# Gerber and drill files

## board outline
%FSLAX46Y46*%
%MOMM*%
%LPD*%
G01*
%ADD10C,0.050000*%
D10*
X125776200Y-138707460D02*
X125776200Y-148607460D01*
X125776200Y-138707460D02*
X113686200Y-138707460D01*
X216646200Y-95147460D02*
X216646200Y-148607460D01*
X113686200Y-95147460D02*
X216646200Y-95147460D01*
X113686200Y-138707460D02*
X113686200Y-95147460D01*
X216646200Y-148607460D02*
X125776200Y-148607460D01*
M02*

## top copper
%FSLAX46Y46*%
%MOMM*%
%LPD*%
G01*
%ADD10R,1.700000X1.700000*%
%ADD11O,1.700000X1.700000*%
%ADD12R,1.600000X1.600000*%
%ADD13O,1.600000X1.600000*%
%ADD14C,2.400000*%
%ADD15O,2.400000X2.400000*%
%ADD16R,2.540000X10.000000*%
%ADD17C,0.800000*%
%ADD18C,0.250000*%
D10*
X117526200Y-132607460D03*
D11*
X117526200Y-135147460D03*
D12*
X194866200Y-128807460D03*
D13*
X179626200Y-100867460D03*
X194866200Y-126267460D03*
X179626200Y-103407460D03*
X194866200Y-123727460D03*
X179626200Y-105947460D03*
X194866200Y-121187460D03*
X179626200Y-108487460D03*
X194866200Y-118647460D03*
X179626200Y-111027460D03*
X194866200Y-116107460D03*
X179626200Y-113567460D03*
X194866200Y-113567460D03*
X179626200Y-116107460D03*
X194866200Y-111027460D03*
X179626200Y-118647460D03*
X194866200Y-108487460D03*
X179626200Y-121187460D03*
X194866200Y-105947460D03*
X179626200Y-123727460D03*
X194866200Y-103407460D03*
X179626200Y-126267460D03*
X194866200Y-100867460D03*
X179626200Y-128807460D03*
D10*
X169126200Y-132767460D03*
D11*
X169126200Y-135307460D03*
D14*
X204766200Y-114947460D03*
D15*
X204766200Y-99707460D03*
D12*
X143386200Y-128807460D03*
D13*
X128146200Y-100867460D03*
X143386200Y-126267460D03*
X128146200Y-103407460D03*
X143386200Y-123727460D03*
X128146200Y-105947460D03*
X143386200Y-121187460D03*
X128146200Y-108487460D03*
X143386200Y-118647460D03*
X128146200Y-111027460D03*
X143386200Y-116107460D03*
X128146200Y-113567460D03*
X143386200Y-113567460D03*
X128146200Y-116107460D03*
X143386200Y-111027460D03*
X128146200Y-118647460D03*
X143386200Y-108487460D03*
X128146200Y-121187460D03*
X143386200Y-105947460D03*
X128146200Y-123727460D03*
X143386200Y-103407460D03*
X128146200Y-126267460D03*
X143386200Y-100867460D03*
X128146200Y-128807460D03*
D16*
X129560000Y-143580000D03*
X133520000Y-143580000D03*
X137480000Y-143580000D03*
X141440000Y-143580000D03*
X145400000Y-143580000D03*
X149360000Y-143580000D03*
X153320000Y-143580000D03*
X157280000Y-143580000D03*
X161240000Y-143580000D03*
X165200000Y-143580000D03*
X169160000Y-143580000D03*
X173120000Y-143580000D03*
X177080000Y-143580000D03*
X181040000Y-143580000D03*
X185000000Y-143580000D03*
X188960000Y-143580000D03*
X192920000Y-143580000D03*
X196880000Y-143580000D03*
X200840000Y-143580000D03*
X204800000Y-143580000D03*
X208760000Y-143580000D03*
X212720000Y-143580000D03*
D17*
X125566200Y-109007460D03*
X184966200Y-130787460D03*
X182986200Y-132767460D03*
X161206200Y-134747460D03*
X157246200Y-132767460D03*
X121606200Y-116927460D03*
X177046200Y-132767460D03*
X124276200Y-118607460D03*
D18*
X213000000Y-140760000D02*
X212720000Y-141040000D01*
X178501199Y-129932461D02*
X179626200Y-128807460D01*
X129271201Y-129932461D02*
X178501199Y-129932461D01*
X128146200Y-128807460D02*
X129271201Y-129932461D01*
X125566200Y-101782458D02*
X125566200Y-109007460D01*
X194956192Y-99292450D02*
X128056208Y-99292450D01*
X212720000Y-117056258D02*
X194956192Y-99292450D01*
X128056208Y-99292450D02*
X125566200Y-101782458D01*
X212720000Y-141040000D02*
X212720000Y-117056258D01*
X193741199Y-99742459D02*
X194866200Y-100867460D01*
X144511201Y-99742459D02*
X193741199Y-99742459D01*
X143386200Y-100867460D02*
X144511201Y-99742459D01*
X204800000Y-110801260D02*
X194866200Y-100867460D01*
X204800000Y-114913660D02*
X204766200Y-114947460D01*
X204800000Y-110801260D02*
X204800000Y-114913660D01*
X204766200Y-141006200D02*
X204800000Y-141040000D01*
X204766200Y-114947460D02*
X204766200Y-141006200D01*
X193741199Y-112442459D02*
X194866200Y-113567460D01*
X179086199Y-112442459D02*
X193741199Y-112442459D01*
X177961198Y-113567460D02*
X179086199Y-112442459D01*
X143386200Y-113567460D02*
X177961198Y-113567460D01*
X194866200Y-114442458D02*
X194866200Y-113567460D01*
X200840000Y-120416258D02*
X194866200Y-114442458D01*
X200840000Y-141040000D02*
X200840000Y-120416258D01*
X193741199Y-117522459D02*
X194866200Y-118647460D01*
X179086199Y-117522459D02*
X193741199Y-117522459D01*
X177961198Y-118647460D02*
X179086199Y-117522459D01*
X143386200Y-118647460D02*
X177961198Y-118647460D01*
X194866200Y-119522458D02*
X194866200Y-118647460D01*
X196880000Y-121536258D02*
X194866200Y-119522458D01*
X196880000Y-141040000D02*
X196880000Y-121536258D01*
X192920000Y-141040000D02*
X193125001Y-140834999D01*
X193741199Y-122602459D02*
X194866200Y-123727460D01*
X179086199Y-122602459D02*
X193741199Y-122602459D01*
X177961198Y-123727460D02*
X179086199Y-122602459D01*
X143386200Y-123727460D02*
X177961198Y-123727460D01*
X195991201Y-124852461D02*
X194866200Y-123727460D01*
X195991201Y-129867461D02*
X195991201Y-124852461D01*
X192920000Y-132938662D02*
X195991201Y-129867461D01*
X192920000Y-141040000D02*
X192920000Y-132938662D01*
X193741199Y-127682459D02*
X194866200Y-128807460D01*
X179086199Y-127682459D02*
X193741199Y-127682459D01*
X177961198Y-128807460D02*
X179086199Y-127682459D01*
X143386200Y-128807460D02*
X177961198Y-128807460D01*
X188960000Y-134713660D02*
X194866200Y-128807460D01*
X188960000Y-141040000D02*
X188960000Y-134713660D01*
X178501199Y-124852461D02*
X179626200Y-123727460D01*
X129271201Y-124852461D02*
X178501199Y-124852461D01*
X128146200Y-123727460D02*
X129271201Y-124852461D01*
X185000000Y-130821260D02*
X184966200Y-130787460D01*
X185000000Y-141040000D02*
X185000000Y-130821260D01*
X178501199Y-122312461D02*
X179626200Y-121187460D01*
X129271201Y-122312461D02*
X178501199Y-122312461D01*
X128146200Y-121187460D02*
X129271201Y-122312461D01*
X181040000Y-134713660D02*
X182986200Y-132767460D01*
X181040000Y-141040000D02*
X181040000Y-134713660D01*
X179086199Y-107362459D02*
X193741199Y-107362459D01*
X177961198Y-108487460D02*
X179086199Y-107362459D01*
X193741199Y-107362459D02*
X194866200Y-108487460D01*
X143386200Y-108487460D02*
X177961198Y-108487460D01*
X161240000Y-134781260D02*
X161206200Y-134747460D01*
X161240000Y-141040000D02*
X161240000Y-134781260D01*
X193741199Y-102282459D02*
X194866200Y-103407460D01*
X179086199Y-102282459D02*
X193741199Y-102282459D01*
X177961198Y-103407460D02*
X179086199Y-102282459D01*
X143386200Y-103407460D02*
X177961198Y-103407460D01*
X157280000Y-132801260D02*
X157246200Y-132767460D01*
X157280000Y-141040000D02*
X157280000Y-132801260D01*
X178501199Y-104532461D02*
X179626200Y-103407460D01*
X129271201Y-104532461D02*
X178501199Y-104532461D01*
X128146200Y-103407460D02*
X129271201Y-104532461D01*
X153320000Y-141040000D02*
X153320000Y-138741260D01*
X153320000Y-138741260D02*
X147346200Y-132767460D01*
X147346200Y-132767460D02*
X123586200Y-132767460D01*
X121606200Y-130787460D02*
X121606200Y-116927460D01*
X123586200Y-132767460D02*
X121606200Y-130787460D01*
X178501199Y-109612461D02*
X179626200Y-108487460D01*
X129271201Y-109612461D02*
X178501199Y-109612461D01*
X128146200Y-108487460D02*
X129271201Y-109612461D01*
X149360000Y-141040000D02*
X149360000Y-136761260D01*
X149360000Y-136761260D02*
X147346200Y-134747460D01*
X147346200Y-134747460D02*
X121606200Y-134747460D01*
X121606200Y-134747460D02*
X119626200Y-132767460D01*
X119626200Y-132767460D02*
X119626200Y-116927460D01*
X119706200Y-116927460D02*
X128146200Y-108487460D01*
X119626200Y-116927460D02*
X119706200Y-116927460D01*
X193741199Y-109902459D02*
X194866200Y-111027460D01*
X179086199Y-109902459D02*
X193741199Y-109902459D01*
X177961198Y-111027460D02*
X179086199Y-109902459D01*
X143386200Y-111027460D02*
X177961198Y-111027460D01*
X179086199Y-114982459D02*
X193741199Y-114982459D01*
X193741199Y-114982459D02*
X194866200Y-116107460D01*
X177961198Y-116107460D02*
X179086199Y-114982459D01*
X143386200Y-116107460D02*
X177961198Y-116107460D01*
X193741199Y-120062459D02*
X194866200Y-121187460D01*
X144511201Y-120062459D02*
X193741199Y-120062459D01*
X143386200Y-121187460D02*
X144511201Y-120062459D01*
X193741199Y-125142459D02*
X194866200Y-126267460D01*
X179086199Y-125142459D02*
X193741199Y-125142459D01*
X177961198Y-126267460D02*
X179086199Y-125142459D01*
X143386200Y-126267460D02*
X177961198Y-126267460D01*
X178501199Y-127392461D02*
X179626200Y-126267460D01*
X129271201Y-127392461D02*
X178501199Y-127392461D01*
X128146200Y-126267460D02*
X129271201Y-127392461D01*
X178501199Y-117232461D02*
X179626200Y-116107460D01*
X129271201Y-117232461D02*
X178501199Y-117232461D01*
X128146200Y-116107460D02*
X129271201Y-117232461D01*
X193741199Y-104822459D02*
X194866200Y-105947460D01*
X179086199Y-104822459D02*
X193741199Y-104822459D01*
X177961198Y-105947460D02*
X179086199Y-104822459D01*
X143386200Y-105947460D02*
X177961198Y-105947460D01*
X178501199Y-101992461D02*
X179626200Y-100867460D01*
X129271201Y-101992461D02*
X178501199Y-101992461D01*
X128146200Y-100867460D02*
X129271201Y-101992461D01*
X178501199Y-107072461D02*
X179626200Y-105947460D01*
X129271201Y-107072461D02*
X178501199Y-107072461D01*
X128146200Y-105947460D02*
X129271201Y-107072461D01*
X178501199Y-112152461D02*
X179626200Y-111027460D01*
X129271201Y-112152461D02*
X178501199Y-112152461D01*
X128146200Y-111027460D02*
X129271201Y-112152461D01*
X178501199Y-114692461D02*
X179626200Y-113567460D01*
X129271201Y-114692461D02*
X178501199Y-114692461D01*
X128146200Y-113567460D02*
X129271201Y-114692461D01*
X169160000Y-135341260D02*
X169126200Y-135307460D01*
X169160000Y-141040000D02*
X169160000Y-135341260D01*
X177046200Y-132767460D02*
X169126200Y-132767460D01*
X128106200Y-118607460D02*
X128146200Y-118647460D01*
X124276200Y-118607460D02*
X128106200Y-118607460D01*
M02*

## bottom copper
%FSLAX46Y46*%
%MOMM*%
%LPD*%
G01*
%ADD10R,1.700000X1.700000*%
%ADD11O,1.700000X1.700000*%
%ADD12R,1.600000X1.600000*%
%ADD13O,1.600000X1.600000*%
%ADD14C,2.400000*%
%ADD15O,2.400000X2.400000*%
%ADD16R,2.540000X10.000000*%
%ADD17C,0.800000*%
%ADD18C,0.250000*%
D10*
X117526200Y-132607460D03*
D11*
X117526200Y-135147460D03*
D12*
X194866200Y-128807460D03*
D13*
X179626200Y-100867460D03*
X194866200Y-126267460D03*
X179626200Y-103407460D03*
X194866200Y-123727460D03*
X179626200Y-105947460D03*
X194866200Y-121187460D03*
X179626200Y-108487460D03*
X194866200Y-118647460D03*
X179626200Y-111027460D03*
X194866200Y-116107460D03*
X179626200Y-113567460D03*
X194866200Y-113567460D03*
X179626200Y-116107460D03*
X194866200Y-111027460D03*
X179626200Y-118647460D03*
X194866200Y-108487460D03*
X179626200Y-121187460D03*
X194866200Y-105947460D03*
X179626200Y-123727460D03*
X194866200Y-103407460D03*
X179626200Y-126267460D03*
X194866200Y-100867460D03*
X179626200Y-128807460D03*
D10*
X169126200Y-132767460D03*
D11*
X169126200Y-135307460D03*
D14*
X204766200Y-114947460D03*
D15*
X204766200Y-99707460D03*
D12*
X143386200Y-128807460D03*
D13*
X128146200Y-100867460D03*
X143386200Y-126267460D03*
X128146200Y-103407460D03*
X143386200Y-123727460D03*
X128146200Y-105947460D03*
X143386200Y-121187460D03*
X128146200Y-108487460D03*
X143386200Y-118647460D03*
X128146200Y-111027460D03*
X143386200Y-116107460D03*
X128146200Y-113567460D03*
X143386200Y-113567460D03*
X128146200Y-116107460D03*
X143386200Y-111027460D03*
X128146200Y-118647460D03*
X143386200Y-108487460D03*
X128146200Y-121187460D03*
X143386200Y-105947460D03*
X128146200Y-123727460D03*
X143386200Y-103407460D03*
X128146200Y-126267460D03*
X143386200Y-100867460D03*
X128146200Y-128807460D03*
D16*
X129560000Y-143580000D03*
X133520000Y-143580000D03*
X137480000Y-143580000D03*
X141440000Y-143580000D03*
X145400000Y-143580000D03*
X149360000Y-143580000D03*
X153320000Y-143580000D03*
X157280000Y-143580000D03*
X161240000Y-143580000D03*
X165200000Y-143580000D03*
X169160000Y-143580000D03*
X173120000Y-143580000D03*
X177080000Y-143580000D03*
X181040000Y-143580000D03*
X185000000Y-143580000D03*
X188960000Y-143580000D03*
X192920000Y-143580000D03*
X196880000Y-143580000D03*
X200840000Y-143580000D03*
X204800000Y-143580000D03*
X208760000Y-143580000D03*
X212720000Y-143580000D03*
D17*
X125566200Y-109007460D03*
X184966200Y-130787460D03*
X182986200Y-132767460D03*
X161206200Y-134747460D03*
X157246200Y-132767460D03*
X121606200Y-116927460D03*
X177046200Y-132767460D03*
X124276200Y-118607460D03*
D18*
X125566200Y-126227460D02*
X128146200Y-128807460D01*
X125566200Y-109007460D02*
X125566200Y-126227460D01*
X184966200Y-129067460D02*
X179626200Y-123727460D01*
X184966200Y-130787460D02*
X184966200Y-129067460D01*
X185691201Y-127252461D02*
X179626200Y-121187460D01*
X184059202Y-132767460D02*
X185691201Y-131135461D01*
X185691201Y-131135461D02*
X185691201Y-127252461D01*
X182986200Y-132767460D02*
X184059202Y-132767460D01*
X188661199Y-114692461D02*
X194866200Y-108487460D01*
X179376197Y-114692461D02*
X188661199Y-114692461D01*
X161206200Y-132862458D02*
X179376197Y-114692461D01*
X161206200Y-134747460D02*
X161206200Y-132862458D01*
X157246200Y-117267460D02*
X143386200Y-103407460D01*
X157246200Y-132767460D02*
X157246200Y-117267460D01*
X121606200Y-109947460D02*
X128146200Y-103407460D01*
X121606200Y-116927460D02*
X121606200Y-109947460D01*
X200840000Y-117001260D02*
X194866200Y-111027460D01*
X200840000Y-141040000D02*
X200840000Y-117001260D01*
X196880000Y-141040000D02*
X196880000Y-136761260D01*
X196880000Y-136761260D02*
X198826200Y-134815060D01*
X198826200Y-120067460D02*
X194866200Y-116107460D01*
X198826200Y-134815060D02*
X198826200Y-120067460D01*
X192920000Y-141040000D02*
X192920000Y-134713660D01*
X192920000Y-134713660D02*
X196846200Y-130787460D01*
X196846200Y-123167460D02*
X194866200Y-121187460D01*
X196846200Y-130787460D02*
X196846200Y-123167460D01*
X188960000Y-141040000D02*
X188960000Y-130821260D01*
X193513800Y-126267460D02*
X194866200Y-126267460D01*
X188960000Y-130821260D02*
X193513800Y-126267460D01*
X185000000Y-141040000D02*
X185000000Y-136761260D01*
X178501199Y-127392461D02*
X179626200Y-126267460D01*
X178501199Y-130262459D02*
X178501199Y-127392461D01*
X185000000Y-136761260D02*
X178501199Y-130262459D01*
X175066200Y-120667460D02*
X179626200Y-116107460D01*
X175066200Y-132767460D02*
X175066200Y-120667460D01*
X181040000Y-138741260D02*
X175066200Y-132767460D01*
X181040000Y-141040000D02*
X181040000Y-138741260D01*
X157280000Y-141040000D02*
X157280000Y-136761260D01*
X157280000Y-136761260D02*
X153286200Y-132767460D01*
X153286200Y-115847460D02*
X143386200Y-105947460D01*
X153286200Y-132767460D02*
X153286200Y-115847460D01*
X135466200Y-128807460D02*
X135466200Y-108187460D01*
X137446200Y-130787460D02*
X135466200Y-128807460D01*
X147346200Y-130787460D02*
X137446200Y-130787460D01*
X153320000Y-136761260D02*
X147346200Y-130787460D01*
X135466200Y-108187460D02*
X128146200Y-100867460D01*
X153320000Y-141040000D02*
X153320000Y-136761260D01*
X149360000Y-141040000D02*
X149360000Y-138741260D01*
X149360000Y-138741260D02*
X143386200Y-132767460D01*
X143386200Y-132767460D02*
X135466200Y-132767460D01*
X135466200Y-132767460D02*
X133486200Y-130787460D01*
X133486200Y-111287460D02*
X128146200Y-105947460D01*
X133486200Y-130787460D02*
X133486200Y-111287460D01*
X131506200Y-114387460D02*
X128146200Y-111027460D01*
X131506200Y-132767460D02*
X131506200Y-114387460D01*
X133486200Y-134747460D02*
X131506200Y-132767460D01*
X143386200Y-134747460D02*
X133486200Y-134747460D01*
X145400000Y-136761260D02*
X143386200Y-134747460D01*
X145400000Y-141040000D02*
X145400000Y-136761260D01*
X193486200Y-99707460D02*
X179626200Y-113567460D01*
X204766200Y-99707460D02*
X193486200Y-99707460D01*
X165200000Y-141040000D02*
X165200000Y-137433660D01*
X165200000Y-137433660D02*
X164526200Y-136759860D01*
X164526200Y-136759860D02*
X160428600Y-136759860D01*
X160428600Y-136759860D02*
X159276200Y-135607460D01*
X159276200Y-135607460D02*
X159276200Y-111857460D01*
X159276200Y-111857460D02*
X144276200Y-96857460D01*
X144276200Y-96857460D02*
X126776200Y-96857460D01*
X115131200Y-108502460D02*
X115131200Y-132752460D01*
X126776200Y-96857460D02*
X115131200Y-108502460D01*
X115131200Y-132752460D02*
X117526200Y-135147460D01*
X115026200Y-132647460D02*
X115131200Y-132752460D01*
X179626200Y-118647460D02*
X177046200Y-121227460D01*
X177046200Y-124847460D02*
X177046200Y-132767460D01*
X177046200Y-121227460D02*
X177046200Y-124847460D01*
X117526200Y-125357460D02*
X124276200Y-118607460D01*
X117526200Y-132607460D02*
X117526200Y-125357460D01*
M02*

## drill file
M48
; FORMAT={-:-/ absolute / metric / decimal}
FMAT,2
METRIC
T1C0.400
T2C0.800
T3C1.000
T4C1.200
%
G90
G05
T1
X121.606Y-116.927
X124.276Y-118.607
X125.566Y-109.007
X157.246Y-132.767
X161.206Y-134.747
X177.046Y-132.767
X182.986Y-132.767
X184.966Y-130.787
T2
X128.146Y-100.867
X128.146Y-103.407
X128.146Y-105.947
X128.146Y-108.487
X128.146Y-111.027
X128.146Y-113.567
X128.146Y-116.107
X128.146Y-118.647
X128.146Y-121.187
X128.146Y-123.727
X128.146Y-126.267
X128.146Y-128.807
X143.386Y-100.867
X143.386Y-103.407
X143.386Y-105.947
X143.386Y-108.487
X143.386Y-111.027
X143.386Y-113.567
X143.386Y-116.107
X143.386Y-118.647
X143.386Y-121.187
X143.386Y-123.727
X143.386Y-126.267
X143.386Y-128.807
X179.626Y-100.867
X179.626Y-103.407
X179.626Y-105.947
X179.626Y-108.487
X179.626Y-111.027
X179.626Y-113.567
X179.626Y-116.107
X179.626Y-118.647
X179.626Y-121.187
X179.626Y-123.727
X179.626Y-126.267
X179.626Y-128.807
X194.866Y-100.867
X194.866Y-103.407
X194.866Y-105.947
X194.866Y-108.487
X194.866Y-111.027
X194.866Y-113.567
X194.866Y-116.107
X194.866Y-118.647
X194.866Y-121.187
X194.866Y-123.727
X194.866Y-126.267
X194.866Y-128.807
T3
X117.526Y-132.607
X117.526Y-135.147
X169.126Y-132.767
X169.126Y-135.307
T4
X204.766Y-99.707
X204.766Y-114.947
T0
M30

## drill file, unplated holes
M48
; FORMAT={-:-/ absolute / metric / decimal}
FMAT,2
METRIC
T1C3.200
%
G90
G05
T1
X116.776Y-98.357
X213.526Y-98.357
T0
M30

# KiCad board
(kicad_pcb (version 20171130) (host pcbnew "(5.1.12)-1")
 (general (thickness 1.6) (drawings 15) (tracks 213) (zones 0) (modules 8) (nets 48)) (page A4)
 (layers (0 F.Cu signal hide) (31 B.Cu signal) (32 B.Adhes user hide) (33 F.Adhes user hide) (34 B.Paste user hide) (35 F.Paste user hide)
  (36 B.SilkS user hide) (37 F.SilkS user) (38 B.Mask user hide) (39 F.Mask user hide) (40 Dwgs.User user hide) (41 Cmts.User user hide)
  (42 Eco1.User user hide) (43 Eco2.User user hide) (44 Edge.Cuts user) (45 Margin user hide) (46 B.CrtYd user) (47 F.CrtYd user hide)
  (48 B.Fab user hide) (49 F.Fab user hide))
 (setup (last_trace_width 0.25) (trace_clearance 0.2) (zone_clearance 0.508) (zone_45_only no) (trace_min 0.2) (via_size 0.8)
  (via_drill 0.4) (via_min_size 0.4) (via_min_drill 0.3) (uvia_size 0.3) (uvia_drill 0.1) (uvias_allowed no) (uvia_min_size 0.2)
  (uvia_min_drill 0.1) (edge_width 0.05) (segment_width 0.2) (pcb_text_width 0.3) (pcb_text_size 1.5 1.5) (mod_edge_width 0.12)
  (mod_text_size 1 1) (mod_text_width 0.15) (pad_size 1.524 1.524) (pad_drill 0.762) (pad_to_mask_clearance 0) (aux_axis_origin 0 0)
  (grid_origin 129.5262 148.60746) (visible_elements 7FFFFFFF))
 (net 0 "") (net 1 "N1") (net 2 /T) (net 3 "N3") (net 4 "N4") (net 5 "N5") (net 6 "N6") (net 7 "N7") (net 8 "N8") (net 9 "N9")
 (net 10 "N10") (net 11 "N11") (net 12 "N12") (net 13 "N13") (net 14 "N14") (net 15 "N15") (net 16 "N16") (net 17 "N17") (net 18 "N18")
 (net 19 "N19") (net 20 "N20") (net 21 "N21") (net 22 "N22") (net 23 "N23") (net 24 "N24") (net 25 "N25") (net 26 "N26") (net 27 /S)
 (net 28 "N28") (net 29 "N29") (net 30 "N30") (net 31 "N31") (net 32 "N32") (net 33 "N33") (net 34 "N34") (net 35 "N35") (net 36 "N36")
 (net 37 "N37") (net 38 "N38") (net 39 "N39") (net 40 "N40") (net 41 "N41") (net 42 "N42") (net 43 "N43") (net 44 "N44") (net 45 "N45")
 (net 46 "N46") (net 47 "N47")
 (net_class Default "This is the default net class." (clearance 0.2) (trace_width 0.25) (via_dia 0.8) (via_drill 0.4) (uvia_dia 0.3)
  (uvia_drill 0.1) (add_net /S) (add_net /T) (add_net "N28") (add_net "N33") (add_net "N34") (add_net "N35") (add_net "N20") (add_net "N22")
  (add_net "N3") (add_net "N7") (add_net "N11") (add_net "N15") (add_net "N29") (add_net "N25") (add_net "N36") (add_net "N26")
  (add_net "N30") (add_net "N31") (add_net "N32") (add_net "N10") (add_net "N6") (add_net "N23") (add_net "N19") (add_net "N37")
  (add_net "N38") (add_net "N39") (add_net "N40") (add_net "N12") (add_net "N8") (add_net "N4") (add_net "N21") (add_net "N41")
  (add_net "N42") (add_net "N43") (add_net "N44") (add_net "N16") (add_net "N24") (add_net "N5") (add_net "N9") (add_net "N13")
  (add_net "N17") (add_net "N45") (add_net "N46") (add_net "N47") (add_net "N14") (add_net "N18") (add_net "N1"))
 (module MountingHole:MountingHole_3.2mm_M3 (layer F.Cu) (at 213.5262 98.35746)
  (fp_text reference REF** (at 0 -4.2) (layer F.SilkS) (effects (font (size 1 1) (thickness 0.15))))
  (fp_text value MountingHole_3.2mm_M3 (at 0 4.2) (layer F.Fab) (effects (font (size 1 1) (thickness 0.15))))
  (pad 1 np_thru_hole circle (at 0 0) (size 3.2 3.2) (drill 3.2) (layers *.Cu *.Mask)))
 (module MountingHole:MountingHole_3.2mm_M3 (layer F.Cu) (at 116.7762 98.35746)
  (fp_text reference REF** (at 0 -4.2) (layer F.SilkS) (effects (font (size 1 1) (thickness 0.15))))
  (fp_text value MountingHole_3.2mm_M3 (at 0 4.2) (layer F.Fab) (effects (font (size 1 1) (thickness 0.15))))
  (pad 1 np_thru_hole circle (at 0 0) (size 3.2 3.2) (drill 3.2) (layers *.Cu *.Mask)))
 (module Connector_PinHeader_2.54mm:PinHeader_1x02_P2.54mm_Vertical (layer F.Cu) (at 117.5262 132.60746)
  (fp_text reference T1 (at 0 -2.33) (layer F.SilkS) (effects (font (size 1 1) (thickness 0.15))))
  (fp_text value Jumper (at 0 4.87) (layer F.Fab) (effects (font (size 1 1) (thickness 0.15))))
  (pad 1 thru_hole rect (at 0 0) (size 1.7 1.7) (drill 1) (layers *.Cu *.Mask) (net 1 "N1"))
  (pad 2 thru_hole oval (at 0 2.54) (size 1.7 1.7) (drill 1) (layers *.Cu *.Mask) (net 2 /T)))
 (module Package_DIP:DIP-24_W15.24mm (layer F.Cu) (at 194.8662 128.80746 180)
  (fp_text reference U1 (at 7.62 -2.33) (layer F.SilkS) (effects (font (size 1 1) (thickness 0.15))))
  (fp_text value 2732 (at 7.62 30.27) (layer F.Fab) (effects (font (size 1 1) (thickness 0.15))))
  (pad 1 thru_hole rect (at 0 0 180) (size 1.6 1.6) (drill 0.8) (layers *.Cu *.Mask) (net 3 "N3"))
  (pad 13 thru_hole oval (at 15.24 27.94 180) (size 1.6 1.6) (drill 0.8) (layers *.Cu *.Mask) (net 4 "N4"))
  (pad 2 thru_hole oval (at 0 2.54 180) (size 1.6 1.6) (drill 0.8) (layers *.Cu *.Mask) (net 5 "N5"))
  (pad 14 thru_hole oval (at 15.24 25.4 180) (size 1.6 1.6) (drill 0.8) (layers *.Cu *.Mask) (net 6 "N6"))
  (pad 3 thru_hole oval (at 0 5.08 180) (size 1.6 1.6) (drill 0.8) (layers *.Cu *.Mask) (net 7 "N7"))
  (pad 15 thru_hole oval (at 15.24 22.86 180) (size 1.6 1.6) (drill 0.8) (layers *.Cu *.Mask) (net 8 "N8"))
  (pad 4 thru_hole oval (at 0 7.62 180) (size 1.6 1.6) (drill 0.8) (layers *.Cu *.Mask) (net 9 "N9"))
  (pad 16 thru_hole oval (at 15.24 20.32 180) (size 1.6 1.6) (drill 0.8) (layers *.Cu *.Mask) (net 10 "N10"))
  (pad 5 thru_hole oval (at 0 10.16 180) (size 1.6 1.6) (drill 0.8) (layers *.Cu *.Mask) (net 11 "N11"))
  (pad 17 thru_hole oval (at 15.24 17.78 180) (size 1.6 1.6) (drill 0.8) (layers *.Cu *.Mask) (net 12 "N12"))
  (pad 6 thru_hole oval (at 0 12.7 180) (size 1.6 1.6) (drill 0.8) (layers *.Cu *.Mask) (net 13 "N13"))
  (pad 18 thru_hole oval (at 15.24 15.24 180) (size 1.6 1.6) (drill 0.8) (layers *.Cu *.Mask) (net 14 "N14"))
  (pad 7 thru_hole oval (at 0 15.24 180) (size 1.6 1.6) (drill 0.8) (layers *.Cu *.Mask) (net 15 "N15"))
  (pad 19 thru_hole oval (at 15.24 12.7 180) (size 1.6 1.6) (drill 0.8) (layers *.Cu *.Mask) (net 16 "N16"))
  (pad 8 thru_hole oval (at 0 17.78 180) (size 1.6 1.6) (drill 0.8) (layers *.Cu *.Mask) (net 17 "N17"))
  (pad 20 thru_hole oval (at 15.24 10.16 180) (size 1.6 1.6) (drill 0.8) (layers *.Cu *.Mask) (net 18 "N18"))
  (pad 9 thru_hole oval (at 0 20.32 180) (size 1.6 1.6) (drill 0.8) (layers *.Cu *.Mask) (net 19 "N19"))
  (pad 21 thru_hole oval (at 15.24 7.62 180) (size 1.6 1.6) (drill 0.8) (layers *.Cu *.Mask) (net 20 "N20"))
  (pad 10 thru_hole oval (at 0 22.86 180) (size 1.6 1.6) (drill 0.8) (layers *.Cu *.Mask) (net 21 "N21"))
  (pad 22 thru_hole oval (at 15.24 5.08 180) (size 1.6 1.6) (drill 0.8) (layers *.Cu *.Mask) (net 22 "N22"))
  (pad 11 thru_hole oval (at 0 25.4 180) (size 1.6 1.6) (drill 0.8) (layers *.Cu *.Mask) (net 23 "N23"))
  (pad 23 thru_hole oval (at 15.24 2.54 180) (size 1.6 1.6) (drill 0.8) (layers *.Cu *.Mask) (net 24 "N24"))
  (pad 12 thru_hole oval (at 0 27.94 180) (size 1.6 1.6) (drill 0.8) (layers *.Cu *.Mask) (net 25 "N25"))
  (pad 24 thru_hole oval (at 15.24 0 180) (size 1.6 1.6) (drill 0.8) (layers *.Cu *.Mask) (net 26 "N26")))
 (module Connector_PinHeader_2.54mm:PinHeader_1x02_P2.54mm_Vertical (layer F.Cu) (at 169.1262 132.76746)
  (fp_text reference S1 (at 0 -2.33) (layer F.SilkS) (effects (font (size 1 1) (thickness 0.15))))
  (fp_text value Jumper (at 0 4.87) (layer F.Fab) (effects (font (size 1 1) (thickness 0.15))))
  (pad 1 thru_hole rect (at 0 0) (size 1.7 1.7) (drill 1) (layers *.Cu *.Mask) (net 18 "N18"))
  (pad 2 thru_hole oval (at 0 2.54) (size 1.7 1.7) (drill 1) (layers *.Cu *.Mask) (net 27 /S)))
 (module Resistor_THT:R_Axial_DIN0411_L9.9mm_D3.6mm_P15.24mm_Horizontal (layer F.Cu) (at 204.7662 114.94746 90)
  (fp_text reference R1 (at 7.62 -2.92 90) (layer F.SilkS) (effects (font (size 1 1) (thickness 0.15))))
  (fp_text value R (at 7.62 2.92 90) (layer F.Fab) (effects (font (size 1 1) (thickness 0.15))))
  (pad 1 thru_hole circle (at 0 0 90) (size 2.4 2.4) (drill 1.2) (layers *.Cu *.Mask) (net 25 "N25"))
  (pad 2 thru_hole oval (at 15.24 0 90) (size 2.4 2.4) (drill 1.2) (layers *.Cu *.Mask) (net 14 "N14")))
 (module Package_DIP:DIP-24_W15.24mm (layer F.Cu) (at 143.3862 128.80746 180)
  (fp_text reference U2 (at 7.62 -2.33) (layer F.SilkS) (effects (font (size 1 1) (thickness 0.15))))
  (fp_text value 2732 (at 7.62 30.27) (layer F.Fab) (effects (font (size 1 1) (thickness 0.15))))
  (pad 1 thru_hole rect (at 0 0 180) (size 1.6 1.6) (drill 0.8) (layers *.Cu *.Mask) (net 3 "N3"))
  (pad 13 thru_hole oval (at 15.24 27.94 180) (size 1.6 1.6) (drill 0.8) (layers *.Cu *.Mask) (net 4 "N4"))
  (pad 2 thru_hole oval (at 0 2.54 180) (size 1.6 1.6) (drill 0.8) (layers *.Cu *.Mask) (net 5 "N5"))
  (pad 14 thru_hole oval (at 15.24 25.4 180) (size 1.6 1.6) (drill 0.8) (layers *.Cu *.Mask) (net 6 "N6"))
  (pad 3 thru_hole oval (at 0 5.08 180) (size 1.6 1.6) (drill 0.8) (layers *.Cu *.Mask) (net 7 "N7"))
  (pad 15 thru_hole oval (at 15.24 22.86 180) (size 1.6 1.6) (drill 0.8) (layers *.Cu *.Mask) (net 8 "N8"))
  (pad 4 thru_hole oval (at 0 7.62 180) (size 1.6 1.6) (drill 0.8) (layers *.Cu *.Mask) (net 9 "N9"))
  (pad 16 thru_hole oval (at 15.24 20.32 180) (size 1.6 1.6) (drill 0.8) (layers *.Cu *.Mask) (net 10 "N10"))
  (pad 5 thru_hole oval (at 0 10.16 180) (size 1.6 1.6) (drill 0.8) (layers *.Cu *.Mask) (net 11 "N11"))
  (pad 17 thru_hole oval (at 15.24 17.78 180) (size 1.6 1.6) (drill 0.8) (layers *.Cu *.Mask) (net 12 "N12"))
  (pad 6 thru_hole oval (at 0 12.7 180) (size 1.6 1.6) (drill 0.8) (layers *.Cu *.Mask) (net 13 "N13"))
  (pad 18 thru_hole oval (at 15.24 15.24 180) (size 1.6 1.6) (drill 0.8) (layers *.Cu *.Mask) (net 14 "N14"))
  (pad 7 thru_hole oval (at 0 15.24 180) (size 1.6 1.6) (drill 0.8) (layers *.Cu *.Mask) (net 15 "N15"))
  (pad 19 thru_hole oval (at 15.24 12.7 180) (size 1.6 1.6) (drill 0.8) (layers *.Cu *.Mask) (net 16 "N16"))
  (pad 8 thru_hole oval (at 0 17.78 180) (size 1.6 1.6) (drill 0.8) (layers *.Cu *.Mask) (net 17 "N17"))
  (pad 20 thru_hole oval (at 15.24 10.16 180) (size 1.6 1.6) (drill 0.8) (layers *.Cu *.Mask) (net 1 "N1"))
  (pad 9 thru_hole oval (at 0 20.32 180) (size 1.6 1.6) (drill 0.8) (layers *.Cu *.Mask) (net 19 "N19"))
  (pad 21 thru_hole oval (at 15.24 7.62 180) (size 1.6 1.6) (drill 0.8) (layers *.Cu *.Mask) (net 20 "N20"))
  (pad 10 thru_hole oval (at 0 22.86 180) (size 1.6 1.6) (drill 0.8) (layers *.Cu *.Mask) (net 21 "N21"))
  (pad 22 thru_hole oval (at 15.24 5.08 180) (size 1.6 1.6) (drill 0.8) (layers *.Cu *.Mask) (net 22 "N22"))
  (pad 11 thru_hole oval (at 0 25.4 180) (size 1.6 1.6) (drill 0.8) (layers *.Cu *.Mask) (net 23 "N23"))
  (pad 23 thru_hole oval (at 15.24 2.54 180) (size 1.6 1.6) (drill 0.8) (layers *.Cu *.Mask) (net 24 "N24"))
  (pad 12 thru_hole oval (at 0 27.94 180) (size 1.6 1.6) (drill 0.8) (layers *.Cu *.Mask) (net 25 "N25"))
  (pad 24 thru_hole oval (at 15.24 0 180) (size 1.6 1.6) (drill 0.8) (layers *.Cu *.Mask) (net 26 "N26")))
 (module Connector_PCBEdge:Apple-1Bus (layer F.Cu) (at 185 145)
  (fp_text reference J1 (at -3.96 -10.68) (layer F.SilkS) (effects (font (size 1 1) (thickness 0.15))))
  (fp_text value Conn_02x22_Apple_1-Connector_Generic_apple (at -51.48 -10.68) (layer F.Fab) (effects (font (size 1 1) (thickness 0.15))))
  (pad 1 connect rect (at -55.44 -3.96) (size 2.54 10) (drill (offset 0 2.54)) (layers F.Cu F.Mask) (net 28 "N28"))
  (pad 2 connect rect (at -51.48 -3.96) (size 2.54 10) (drill (offset 0 2.54)) (layers F.Cu F.Mask) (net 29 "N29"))
  (pad 3 connect rect (at -47.52 -3.96) (size 2.54 10) (drill (offset 0 2.54)) (layers F.Cu F.Mask) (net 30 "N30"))
  (pad 4 connect rect (at -43.56 -3.96) (size 2.54 10) (drill (offset 0 2.54)) (layers F.Cu F.Mask) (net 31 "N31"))
  (pad 5 connect rect (at -39.6 -3.96) (size 2.54 10) (drill (offset 0 2.54)) (layers F.Cu F.Mask) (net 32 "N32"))
  (pad 6 connect rect (at -35.64 -3.96) (size 2.54 10) (drill (offset 0 2.54)) (layers F.Cu F.Mask) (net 10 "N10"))
  (pad 7 connect rect (at -31.68 -3.96) (size 2.54 10) (drill (offset 0 2.54)) (layers F.Cu F.Mask) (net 6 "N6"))
  (pad 8 connect rect (at -27.72 -3.96) (size 2.54 10) (drill (offset 0 2.54)) (layers F.Cu F.Mask) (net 23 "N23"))
  (pad 9 connect rect (at -23.76 -3.96) (size 2.54 10) (drill (offset 0 2.54)) (layers F.Cu F.Mask) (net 19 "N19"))
  (pad 10 connect rect (at -19.8 -3.96) (size 2.54 10) (drill (offset 0 2.54)) (layers F.Cu F.Mask) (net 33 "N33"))
  (pad 11 connect rect (at -15.84 -3.96) (size 2.54 10) (drill (offset 0 2.54)) (layers F.Cu F.Mask) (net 27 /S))
  (pad 12 connect rect (at -11.88 -3.96) (size 2.54 10) (drill (offset 0 2.54)) (layers F.Cu F.Mask) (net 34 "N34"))
  (pad 13 connect rect (at -7.92 -3.96) (size 2.54 10) (drill (offset 0 2.54)) (layers F.Cu F.Mask) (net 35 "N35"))
  (pad 14 connect rect (at -3.96 -3.96) (size 2.54 10) (drill (offset 0 2.54)) (layers F.Cu F.Mask) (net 20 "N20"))
  (pad 15 connect rect (at 0 -3.96) (size 2.54 10) (drill (offset 0 2.54)) (layers F.Cu F.Mask) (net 22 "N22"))
  (pad 16 connect rect (at 3.96 -3.96) (size 2.54 10) (drill (offset 0 2.54)) (layers F.Cu F.Mask) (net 3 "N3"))
  (pad 17 connect rect (at 7.92 -3.96) (size 2.54 10) (drill (offset 0 2.54)) (layers F.Cu F.Mask) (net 7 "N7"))
  (pad 18 connect rect (at 11.88 -3.96) (size 2.54 10) (drill (offset 0 2.54)) (layers F.Cu F.Mask) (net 11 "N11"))
  (pad 19 connect rect (at 15.84 -3.96) (size 2.54 10) (drill (offset 0 2.54)) (layers F.Cu F.Mask) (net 15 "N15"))
  (pad 20 connect rect (at 19.8 -3.96) (size 2.54 10) (drill (offset 0 2.54)) (layers F.Cu F.Mask) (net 25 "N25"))
  (pad 21 connect rect (at 23.76 -3.96) (size 2.54 10) (drill (offset 0 2.54)) (layers F.Cu F.Mask) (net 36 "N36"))
  (pad 22 connect rect (at 27.72 -3.96) (size 2.54 10) (drill (offset 0 2.54)) (layers F.Cu F.Mask) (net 26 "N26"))
  (pad A connect rect (at -55.44 -3.96) (size 2.54 10) (drill (offset 0 2.54)) (layers B.Cu B.Mask) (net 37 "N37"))
  (pad B connect rect (at -51.48 -3.96) (size 2.54 10) (drill (offset 0 2.54)) (layers B.Cu B.Mask) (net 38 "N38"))
  (pad C connect rect (at -47.52 -3.96) (size 2.54 10) (drill (offset 0 2.54)) (layers B.Cu B.Mask) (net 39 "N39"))
  (pad D connect rect (at -43.56 -3.96) (size 2.54 10) (drill (offset 0 2.54)) (layers B.Cu B.Mask) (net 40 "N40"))
  (pad E connect rect (at -39.6 -3.96) (size 2.54 10) (drill (offset 0 2.54)) (layers B.Cu B.Mask) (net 12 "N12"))
  (pad F connect rect (at -35.64 -3.96) (size 2.54 10) (drill (offset 0 2.54)) (layers B.Cu B.Mask) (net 8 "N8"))
  (pad H connect rect (at -31.68 -3.96) (size 2.54 10) (drill (offset 0 2.54)) (layers B.Cu B.Mask) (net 4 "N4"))
  (pad J connect rect (at -27.72 -3.96) (size 2.54 10) (drill (offset 0 2.54)) (layers B.Cu B.Mask) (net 21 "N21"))
  (pad K connect rect (at -23.76 -3.96) (size 2.54 10) (drill (offset 0 2.54)) (layers B.Cu B.Mask) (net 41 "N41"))
  (pad L connect rect (at -19.8 -3.96) (size 2.54 10) (drill (offset 0 2.54)) (layers B.Cu B.Mask) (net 2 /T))
  (pad M connect rect (at -15.84 -3.96) (size 2.54 10) (drill (offset 0 2.54)) (layers B.Cu B.Mask) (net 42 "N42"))
  (pad N connect rect (at -11.88 -3.96) (size 2.54 10) (drill (offset 0 2.54)) (layers B.Cu B.Mask) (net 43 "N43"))
  (pad P connect rect (at -7.92 -3.96) (size 2.54 10) (drill (offset 0 2.54)) (layers B.Cu B.Mask) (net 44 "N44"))
  (pad R connect rect (at -3.96 -3.96) (size 2.54 10) (drill (offset 0 2.54)) (layers B.Cu B.Mask) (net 16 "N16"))
  (pad S connect rect (at 0 -3.96) (size 2.54 10) (drill (offset 0 2.54)) (layers B.Cu B.Mask) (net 24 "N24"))
  (pad T connect rect (at 3.96 -3.96) (size 2.54 10) (drill (offset 0 2.54)) (layers B.Cu B.Mask) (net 5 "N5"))
  (pad U connect rect (at 7.92 -3.96) (size 2.54 10) (drill (offset 0 2.54)) (layers B.Cu B.Mask) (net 9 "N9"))
  (pad V connect rect (at 11.88 -3.96) (size 2.54 10) (drill (offset 0 2.54)) (layers B.Cu B.Mask) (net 13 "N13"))
  (pad W connect rect (at 15.84 -3.96) (size 2.54 10) (drill (offset 0 2.54)) (layers B.Cu B.Mask) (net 17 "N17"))
  (pad X connect rect (at 19.8 -3.96) (size 2.54 10) (drill (offset 0 2.54)) (layers B.Cu B.Mask) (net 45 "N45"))
  (pad Y connect rect (at 23.76 -3.96) (size 2.54 10) (drill (offset 0 2.54)) (layers B.Cu B.Mask) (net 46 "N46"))
  (pad Z connect rect (at 27.72 -3.96) (size 2.54 10) (drill (offset 0 2.54)) (layers B.Cu B.Mask) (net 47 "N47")))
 (gr_line (start 125.7762 138.70746) (end 125.7762 148.60746) (layer Edge.Cuts) (width 0.05))
 (gr_line (start 125.7762 138.70746) (end 113.6862 138.70746) (layer Edge.Cuts) (width 0.05))
 (gr_line (start 216.6462 95.14746) (end 216.6462 148.60746) (layer Edge.Cuts) (width 0.05))
 (gr_line (start 113.6862 95.14746) (end 216.6462 95.14746) (layer Edge.Cuts) (width 0.05))
 (gr_line (start 113.6862 138.70746) (end 113.6862 95.14746) (layer Edge.Cuts) (width 0.05))
 (gr_line (start 216.6462 148.60746) (end 125.7762 148.60746) (layer Edge.Cuts) (width 0.05))
 (segment (start 213 140.76) (end 212.72 141.04) (width 0.25) (layer F.Cu) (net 26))
 (segment (start 178.501199 129.932461) (end 179.6262 128.80746) (width 0.25) (layer F.Cu) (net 26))
 (segment (start 129.271201 129.932461) (end 178.501199 129.932461) (width 0.25) (layer F.Cu) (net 26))
 (segment (start 128.1462 128.80746) (end 129.271201 129.932461) (width 0.25) (layer F.Cu) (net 26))
 (via (at 125.5662 109.00746) (size 0.8) (drill 0.4) (layers F.Cu B.Cu) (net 26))
 (segment (start 125.5662 101.782458) (end 125.5662 109.00746) (width 0.25) (layer F.Cu) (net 26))
 (segment (start 194.956192 99.29245) (end 128.056208 99.29245) (width 0.25) (layer F.Cu) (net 26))
 (segment (start 212.72 117.056258) (end 194.956192 99.29245) (width 0.25) (layer F.Cu) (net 26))
 (segment (start 128.056208 99.29245) (end 125.5662 101.782458) (width 0.25) (layer F.Cu) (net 26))
 (segment (start 212.72 141.04) (end 212.72 117.056258) (width 0.25) (layer F.Cu) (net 26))
 (segment (start 125.5662 126.22746) (end 128.1462 128.80746) (width 0.25) (layer B.Cu) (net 26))
 (segment (start 125.5662 109.00746) (end 125.5662 126.22746) (width 0.25) (layer B.Cu) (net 26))
 (segment (start 193.741199 99.742459) (end 194.8662 100.86746) (width 0.25) (layer F.Cu) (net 25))
 (segment (start 144.511201 99.742459) (end 193.741199 99.742459) (width 0.25) (layer F.Cu) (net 25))
 (segment (start 143.3862 100.86746) (end 144.511201 99.742459) (width 0.25) (layer F.Cu) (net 25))
 (segment (start 204.8 110.80126) (end 194.8662 100.86746) (width 0.25) (layer F.Cu) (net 25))
 (segment (start 204.8 114.91366) (end 204.7662 114.94746) (width 0.25) (layer F.Cu) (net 25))
 (segment (start 204.8 110.80126) (end 204.8 114.91366) (width 0.25) (layer F.Cu) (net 25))
 (segment (start 204.7662 141.0062) (end 204.8 141.04) (width 0.25) (layer F.Cu) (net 25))
 (segment (start 204.7662 114.94746) (end 204.7662 141.0062) (width 0.25) (layer F.Cu) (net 25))
 (segment (start 193.741199 112.442459) (end 194.8662 113.56746) (width 0.25) (layer F.Cu) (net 15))
 (segment (start 179.086199 112.442459) (end 193.741199 112.442459) (width 0.25) (layer F.Cu) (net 15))
 (segment (start 177.961198 113.56746) (end 179.086199 112.442459) (width 0.25) (layer F.Cu) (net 15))
 (segment (start 143.3862 113.56746) (end 177.961198 113.56746) (width 0.25) (layer F.Cu) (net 15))
 (segment (start 194.8662 114.442458) (end 194.8662 113.56746) (width 0.25) (layer F.Cu) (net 15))
 (segment (start 200.84 120.416258) (end 194.8662 114.442458) (width 0.25) (layer F.Cu) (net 15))
 (segment (start 200.84 141.04) (end 200.84 120.416258) (width 0.25) (layer F.Cu) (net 15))
 (segment (start 193.741199 117.522459) (end 194.8662 118.64746) (width 0.25) (layer F.Cu) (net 11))
 (segment (start 179.086199 117.522459) (end 193.741199 117.522459) (width 0.25) (layer F.Cu) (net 11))
 (segment (start 177.961198 118.64746) (end 179.086199 117.522459) (width 0.25) (layer F.Cu) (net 11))
 (segment (start 143.3862 118.64746) (end 177.961198 118.64746) (width 0.25) (layer F.Cu) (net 11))
 (segment (start 194.8662 119.522458) (end 194.8662 118.64746) (width 0.25) (layer F.Cu) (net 11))
 (segment (start 196.88 121.536258) (end 194.8662 119.522458) (width 0.25) (layer F.Cu) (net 11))
 (segment (start 196.88 141.04) (end 196.88 121.536258) (width 0.25) (layer F.Cu) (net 11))
 (segment (start 192.92 141.04) (end 193.125001 140.834999) (width 0.25) (layer F.Cu) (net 7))
 (segment (start 193.741199 122.602459) (end 194.8662 123.72746) (width 0.25) (layer F.Cu) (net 7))
 (segment (start 179.086199 122.602459) (end 193.741199 122.602459) (width 0.25) (layer F.Cu) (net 7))
 (segment (start 177.961198 123.72746) (end 179.086199 122.602459) (width 0.25) (layer F.Cu) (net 7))
 (segment (start 143.3862 123.72746) (end 177.961198 123.72746) (width 0.25) (layer F.Cu) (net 7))
 (segment (start 195.991201 124.852461) (end 194.8662 123.72746) (width 0.25) (layer F.Cu) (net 7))
 (segment (start 195.991201 129.867461) (end 195.991201 124.852461) (width 0.25) (layer F.Cu) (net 7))
 (segment (start 192.92 132.938662) (end 195.991201 129.867461) (width 0.25) (layer F.Cu) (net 7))
 (segment (start 192.92 141.04) (end 192.92 132.938662) (width 0.25) (layer F.Cu) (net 7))
 (segment (start 193.741199 127.682459) (end 194.8662 128.80746) (width 0.25) (layer F.Cu) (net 3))
 (segment (start 179.086199 127.682459) (end 193.741199 127.682459) (width 0.25) (layer F.Cu) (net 3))
 (segment (start 177.961198 128.80746) (end 179.086199 127.682459) (width 0.25) (layer F.Cu) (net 3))
 (segment (start 143.3862 128.80746) (end 177.961198 128.80746) (width 0.25) (layer F.Cu) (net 3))
 (segment (start 188.96 134.71366) (end 194.8662 128.80746) (width 0.25) (layer F.Cu) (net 3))
 (segment (start 188.96 141.04) (end 188.96 134.71366) (width 0.25) (layer F.Cu) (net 3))
 (segment (start 178.501199 124.852461) (end 179.6262 123.72746) (width 0.25) (layer F.Cu) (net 22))
 (segment (start 129.271201 124.852461) (end 178.501199 124.852461) (width 0.25) (layer F.Cu) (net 22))
 (segment (start 128.1462 123.72746) (end 129.271201 124.852461) (width 0.25) (layer F.Cu) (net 22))
 (via (at 184.9662 130.78746) (size 0.8) (drill 0.4) (layers F.Cu B.Cu) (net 22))
 (segment (start 185 130.82126) (end 184.9662 130.78746) (width 0.25) (layer F.Cu) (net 22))
 (segment (start 185 141.04) (end 185 130.82126) (width 0.25) (layer F.Cu) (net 22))
 (segment (start 184.9662 129.06746) (end 179.6262 123.72746) (width 0.25) (layer B.Cu) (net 22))
 (segment (start 184.9662 130.78746) (end 184.9662 129.06746) (width 0.25) (layer B.Cu) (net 22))
 (segment (start 178.501199 122.312461) (end 179.6262 121.18746) (width 0.25) (layer F.Cu) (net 20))
 (segment (start 129.271201 122.312461) (end 178.501199 122.312461) (width 0.25) (layer F.Cu) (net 20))
 (segment (start 128.1462 121.18746) (end 129.271201 122.312461) (width 0.25) (layer F.Cu) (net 20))
 (via (at 182.9862 132.76746) (size 0.8) (drill 0.4) (layers F.Cu B.Cu) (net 20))
 (segment (start 181.04 134.71366) (end 182.9862 132.76746) (width 0.25) (layer F.Cu) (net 20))
 (segment (start 181.04 141.04) (end 181.04 134.71366) (width 0.25) (layer F.Cu) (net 20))
 (segment (start 185.691201 127.252461) (end 179.6262 121.18746) (width 0.25) (layer B.Cu) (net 20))
 (segment (start 184.059202 132.76746) (end 185.691201 131.135461) (width 0.25) (layer B.Cu) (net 20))
 (segment (start 185.691201 131.135461) (end 185.691201 127.252461) (width 0.25) (layer B.Cu) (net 20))
 (segment (start 182.9862 132.76746) (end 184.059202 132.76746) (width 0.25) (layer B.Cu) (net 20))
 (segment (start 179.086199 107.362459) (end 193.741199 107.362459) (width 0.25) (layer F.Cu) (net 19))
 (segment (start 177.961198 108.48746) (end 179.086199 107.362459) (width 0.25) (layer F.Cu) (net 19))
 (segment (start 193.741199 107.362459) (end 194.8662 108.48746) (width 0.25) (layer F.Cu) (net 19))
 (segment (start 143.3862 108.48746) (end 177.961198 108.48746) (width 0.25) (layer F.Cu) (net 19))
 (via (at 161.2062 134.74746) (size 0.8) (drill 0.4) (layers F.Cu B.Cu) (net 19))
 (segment (start 161.24 134.78126) (end 161.2062 134.74746) (width 0.25) (layer F.Cu) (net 19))
 (segment (start 161.24 141.04) (end 161.24 134.78126) (width 0.25) (layer F.Cu) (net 19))
 (segment (start 188.661199 114.692461) (end 194.8662 108.48746) (width 0.25) (layer B.Cu) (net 19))
 (segment (start 179.376197 114.692461) (end 188.661199 114.692461) (width 0.25) (layer B.Cu) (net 19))
 (segment (start 161.2062 132.862458) (end 179.376197 114.692461) (width 0.25) (layer B.Cu) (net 19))
 (segment (start 161.2062 134.74746) (end 161.2062 132.862458) (width 0.25) (layer B.Cu) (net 19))
 (segment (start 193.741199 102.282459) (end 194.8662 103.40746) (width 0.25) (layer F.Cu) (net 23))
 (segment (start 179.086199 102.282459) (end 193.741199 102.282459) (width 0.25) (layer F.Cu) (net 23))
 (segment (start 177.961198 103.40746) (end 179.086199 102.282459) (width 0.25) (layer F.Cu) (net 23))
 (segment (start 143.3862 103.40746) (end 177.961198 103.40746) (width 0.25) (layer F.Cu) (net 23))
 (via (at 157.2462 132.76746) (size 0.8) (drill 0.4) (layers F.Cu B.Cu) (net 23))
 (segment (start 157.28 132.80126) (end 157.2462 132.76746) (width 0.25) (layer F.Cu) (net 23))
 (segment (start 157.28 141.04) (end 157.28 132.80126) (width 0.25) (layer F.Cu) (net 23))
 (segment (start 157.2462 117.26746) (end 143.3862 103.40746) (width 0.25) (layer B.Cu) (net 23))
 (segment (start 157.2462 132.76746) (end 157.2462 117.26746) (width 0.25) (layer B.Cu) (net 23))
 (segment (start 178.501199 104.532461) (end 179.6262 103.40746) (width 0.25) (layer F.Cu) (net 6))
 (segment (start 129.271201 104.532461) (end 178.501199 104.532461) (width 0.25) (layer F.Cu) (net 6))
 (segment (start 128.1462 103.40746) (end 129.271201 104.532461) (width 0.25) (layer F.Cu) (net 6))
 (segment (start 153.32 141.04) (end 153.32 138.74126) (width 0.25) (layer F.Cu) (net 6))
 (segment (start 153.32 138.74126) (end 147.3462 132.76746) (width 0.25) (layer F.Cu) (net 6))
 (segment (start 147.3462 132.76746) (end 123.5862 132.76746) (width 0.25) (layer F.Cu) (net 6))
 (via (at 121.6062 116.92746) (size 0.8) (drill 0.4) (layers F.Cu B.Cu) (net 6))
 (segment (start 121.6062 130.78746) (end 121.6062 116.92746) (width 0.25) (layer F.Cu) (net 6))
 (segment (start 123.5862 132.76746) (end 121.6062 130.78746) (width 0.25) (layer F.Cu) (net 6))
 (segment (start 121.6062 109.94746) (end 128.1462 103.40746) (width 0.25) (layer B.Cu) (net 6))
 (segment (start 121.6062 116.92746) (end 121.6062 109.94746) (width 0.25) (layer B.Cu) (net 6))
 (segment (start 178.501199 109.612461) (end 179.6262 108.48746) (width 0.25) (layer F.Cu) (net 10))
 (segment (start 129.271201 109.612461) (end 178.501199 109.612461) (width 0.25) (layer F.Cu) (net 10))
 (segment (start 128.1462 108.48746) (end 129.271201 109.612461) (width 0.25) (layer F.Cu) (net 10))
 (segment (start 149.36 141.04) (end 149.36 136.76126) (width 0.25) (layer F.Cu) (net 10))
 (segment (start 149.36 136.76126) (end 147.3462 134.74746) (width 0.25) (layer F.Cu) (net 10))
 (segment (start 147.3462 134.74746) (end 121.6062 134.74746) (width 0.25) (layer F.Cu) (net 10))
 (segment (start 121.6062 134.74746) (end 119.6262 132.76746) (width 0.25) (layer F.Cu) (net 10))
 (segment (start 119.6262 132.76746) (end 119.6262 116.92746) (width 0.25) (layer F.Cu) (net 10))
 (segment (start 119.7062 116.92746) (end 128.1462 108.48746) (width 0.25) (layer F.Cu) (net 10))
 (segment (start 119.6262 116.92746) (end 119.7062 116.92746) (width 0.25) (layer F.Cu) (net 10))
 (segment (start 193.741199 109.902459) (end 194.8662 111.02746) (width 0.25) (layer F.Cu) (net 17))
 (segment (start 179.086199 109.902459) (end 193.741199 109.902459) (width 0.25) (layer F.Cu) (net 17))
 (segment (start 177.961198 111.02746) (end 179.086199 109.902459) (width 0.25) (layer F.Cu) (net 17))
 (segment (start 143.3862 111.02746) (end 177.961198 111.02746) (width 0.25) (layer F.Cu) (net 17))
 (segment (start 200.84 117.00126) (end 194.8662 111.02746) (width 0.25) (layer B.Cu) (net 17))
 (segment (start 200.84 141.04) (end 200.84 117.00126) (width 0.25) (layer B.Cu) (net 17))
 (segment (start 179.086199 114.982459) (end 193.741199 114.982459) (width 0.25) (layer F.Cu) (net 13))
 (segment (start 193.741199 114.982459) (end 194.8662 116.10746) (width 0.25) (layer F.Cu) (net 13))
 (segment (start 177.961198 116.10746) (end 179.086199 114.982459) (width 0.25) (layer F.Cu) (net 13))
 (segment (start 143.3862 116.10746) (end 177.961198 116.10746) (width 0.25) (layer F.Cu) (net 13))
 (segment (start 196.88 141.04) (end 196.88 136.76126) (width 0.25) (layer B.Cu) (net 13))
 (segment (start 196.88 136.76126) (end 198.8262 134.81506) (width 0.25) (layer B.Cu) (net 13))
 (segment (start 198.8262 120.06746) (end 194.8662 116.10746) (width 0.25) (layer B.Cu) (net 13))
 (segment (start 198.8262 134.81506) (end 198.8262 120.06746) (width 0.25) (layer B.Cu) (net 13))
 (segment (start 193.741199 120.062459) (end 194.8662 121.18746) (width 0.25) (layer F.Cu) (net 9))
 (segment (start 144.511201 120.062459) (end 193.741199 120.062459) (width 0.25) (layer F.Cu) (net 9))
 (segment (start 143.3862 121.18746) (end 144.511201 120.062459) (width 0.25) (layer F.Cu) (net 9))
 (segment (start 192.92 141.04) (end 192.92 134.71366) (width 0.25) (layer B.Cu) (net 9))
 (segment (start 192.92 134.71366) (end 196.8462 130.78746) (width 0.25) (layer B.Cu) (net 9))
 (segment (start 196.8462 123.16746) (end 194.8662 121.18746) (width 0.25) (layer B.Cu) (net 9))
 (segment (start 196.8462 130.78746) (end 196.8462 123.16746) (width 0.25) (layer B.Cu) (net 9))
 (segment (start 193.741199 125.142459) (end 194.8662 126.26746) (width 0.25) (layer F.Cu) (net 5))
 (segment (start 179.086199 125.142459) (end 193.741199 125.142459) (width 0.25) (layer F.Cu) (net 5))
 (segment (start 177.961198 126.26746) (end 179.086199 125.142459) (width 0.25) (layer F.Cu) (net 5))
 (segment (start 143.3862 126.26746) (end 177.961198 126.26746) (width 0.25) (layer F.Cu) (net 5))
 (segment (start 188.96 141.04) (end 188.96 130.82126) (width 0.25) (layer B.Cu) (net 5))
 (segment (start 193.5138 126.26746) (end 194.8662 126.26746) (width 0.25) (layer B.Cu) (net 5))
 (segment (start 188.96 130.82126) (end 193.5138 126.26746) (width 0.25) (layer B.Cu) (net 5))
 (segment (start 178.501199 127.392461) (end 179.6262 126.26746) (width 0.25) (layer F.Cu) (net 24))
 (segment (start 129.271201 127.392461) (end 178.501199 127.392461) (width 0.25) (layer F.Cu) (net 24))
 (segment (start 128.1462 126.26746) (end 129.271201 127.392461) (width 0.25) (layer F.Cu) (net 24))
 (segment (start 185 141.04) (end 185 136.76126) (width 0.25) (layer B.Cu) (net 24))
 (segment (start 178.501199 127.392461) (end 179.6262 126.26746) (width 0.25) (layer B.Cu) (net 24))
 (segment (start 178.501199 130.262459) (end 178.501199 127.392461) (width 0.25) (layer B.Cu) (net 24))
 (segment (start 185 136.76126) (end 178.501199 130.262459) (width 0.25) (layer B.Cu) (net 24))
 (segment (start 178.501199 117.232461) (end 179.6262 116.10746) (width 0.25) (layer F.Cu) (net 16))
 (segment (start 129.271201 117.232461) (end 178.501199 117.232461) (width 0.25) (layer F.Cu) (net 16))
 (segment (start 128.1462 116.10746) (end 129.271201 117.232461) (width 0.25) (layer F.Cu) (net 16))
 (segment (start 175.0662 120.66746) (end 179.6262 116.10746) (width 0.25) (layer B.Cu) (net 16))
 (segment (start 175.0662 132.76746) (end 175.0662 120.66746) (width 0.25) (layer B.Cu) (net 16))
 (segment (start 181.04 138.74126) (end 175.0662 132.76746) (width 0.25) (layer B.Cu) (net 16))
 (segment (start 181.04 141.04) (end 181.04 138.74126) (width 0.25) (layer B.Cu) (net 16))
 (segment (start 193.741199 104.822459) (end 194.8662 105.94746) (width 0.25) (layer F.Cu) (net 21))
 (segment (start 179.086199 104.822459) (end 193.741199 104.822459) (width 0.25) (layer F.Cu) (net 21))
 (segment (start 177.961198 105.94746) (end 179.086199 104.822459) (width 0.25) (layer F.Cu) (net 21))
 (segment (start 143.3862 105.94746) (end 177.961198 105.94746) (width 0.25) (layer F.Cu) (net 21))
 (segment (start 157.28 141.04) (end 157.28 136.76126) (width 0.25) (layer B.Cu) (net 21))
 (segment (start 157.28 136.76126) (end 153.2862 132.76746) (width 0.25) (layer B.Cu) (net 21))
 (segment (start 153.2862 115.84746) (end 143.3862 105.94746) (width 0.25) (layer B.Cu) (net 21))
 (segment (start 153.2862 132.76746) (end 153.2862 115.84746) (width 0.25) (layer B.Cu) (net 21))
 (segment (start 178.501199 101.992461) (end 179.6262 100.86746) (width 0.25) (layer F.Cu) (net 4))
 (segment (start 129.271201 101.992461) (end 178.501199 101.992461) (width 0.25) (layer F.Cu) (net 4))
 (segment (start 128.1462 100.86746) (end 129.271201 101.992461) (width 0.25) (layer F.Cu) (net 4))
 (segment (start 135.4662 128.80746) (end 135.4662 108.18746) (width 0.25) (layer B.Cu) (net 4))
 (segment (start 137.4462 130.78746) (end 135.4662 128.80746) (width 0.25) (layer B.Cu) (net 4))
 (segment (start 147.3462 130.78746) (end 137.4462 130.78746) (width 0.25) (layer B.Cu) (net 4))
 (segment (start 153.32 136.76126) (end 147.3462 130.78746) (width 0.25) (layer B.Cu) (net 4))
 (segment (start 135.4662 108.18746) (end 128.1462 100.86746) (width 0.25) (layer B.Cu) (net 4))
 (segment (start 153.32 141.04) (end 153.32 136.76126) (width 0.25) (layer B.Cu) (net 4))
 (segment (start 178.501199 107.072461) (end 179.6262 105.94746) (width 0.25) (layer F.Cu) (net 8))
 (segment (start 129.271201 107.072461) (end 178.501199 107.072461) (width 0.25) (layer F.Cu) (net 8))
 (segment (start 128.1462 105.94746) (end 129.271201 107.072461) (width 0.25) (layer F.Cu) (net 8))
 (segment (start 149.36 141.04) (end 149.36 138.74126) (width 0.25) (layer B.Cu) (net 8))
 (segment (start 149.36 138.74126) (end 143.3862 132.76746) (width 0.25) (layer B.Cu) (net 8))
 (segment (start 143.3862 132.76746) (end 135.4662 132.76746) (width 0.25) (layer B.Cu) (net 8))
 (segment (start 135.4662 132.76746) (end 133.4862 130.78746) (width 0.25) (layer B.Cu) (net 8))
 (segment (start 133.4862 111.28746) (end 128.1462 105.94746) (width 0.25) (layer B.Cu) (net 8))
 (segment (start 133.4862 130.78746) (end 133.4862 111.28746) (width 0.25) (layer B.Cu) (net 8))
 (segment (start 178.501199 112.152461) (end 179.6262 111.02746) (width 0.25) (layer F.Cu) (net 12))
 (segment (start 129.271201 112.152461) (end 178.501199 112.152461) (width 0.25) (layer F.Cu) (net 12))
 (segment (start 128.1462 111.02746) (end 129.271201 112.152461) (width 0.25) (layer F.Cu) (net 12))
 (segment (start 131.5062 114.38746) (end 128.1462 111.02746) (width 0.25) (layer B.Cu) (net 12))
 (segment (start 131.5062 132.76746) (end 131.5062 114.38746) (width 0.25) (layer B.Cu) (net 12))
 (segment (start 133.4862 134.74746) (end 131.5062 132.76746) (width 0.25) (layer B.Cu) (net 12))
 (segment (start 143.3862 134.74746) (end 133.4862 134.74746) (width 0.25) (layer B.Cu) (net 12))
 (segment (start 145.4 136.76126) (end 143.3862 134.74746) (width 0.25) (layer B.Cu) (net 12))
 (segment (start 145.4 141.04) (end 145.4 136.76126) (width 0.25) (layer B.Cu) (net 12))
 (segment (start 178.501199 114.692461) (end 179.6262 113.56746) (width 0.25) (layer F.Cu) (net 14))
 (segment (start 129.271201 114.692461) (end 178.501199 114.692461) (width 0.25) (layer F.Cu) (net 14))
 (segment (start 128.1462 113.56746) (end 129.271201 114.692461) (width 0.25) (layer F.Cu) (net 14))
 (segment (start 193.4862 99.70746) (end 179.6262 113.56746) (width 0.25) (layer B.Cu) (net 14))
 (segment (start 204.7662 99.70746) (end 193.4862 99.70746) (width 0.25) (layer B.Cu) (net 14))
 (segment (start 169.16 135.34126) (end 169.1262 135.30746) (width 0.25) (layer F.Cu) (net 27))
 (segment (start 169.16 141.04) (end 169.16 135.34126) (width 0.25) (layer F.Cu) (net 27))
 (segment (start 165.2 141.04) (end 165.2 137.43366) (width 0.25) (layer B.Cu) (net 2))
 (segment (start 165.2 137.43366) (end 164.5262 136.75986) (width 0.25) (layer B.Cu) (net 2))
 (segment (start 164.5262 136.75986) (end 160.4286 136.75986) (width 0.25) (layer B.Cu) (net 2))
 (segment (start 160.4286 136.75986) (end 159.2762 135.60746) (width 0.25) (layer B.Cu) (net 2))
 (segment (start 159.2762 135.60746) (end 159.2762 111.85746) (width 0.25) (layer B.Cu) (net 2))
 (segment (start 159.2762 111.85746) (end 144.2762 96.85746) (width 0.25) (layer B.Cu) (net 2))
 (segment (start 144.2762 96.85746) (end 126.7762 96.85746) (width 0.25) (layer B.Cu) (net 2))
 (segment (start 115.1312 108.50246) (end 115.1312 132.75246) (width 0.25) (layer B.Cu) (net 2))
 (segment (start 126.7762 96.85746) (end 115.1312 108.50246) (width 0.25) (layer B.Cu) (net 2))
 (segment (start 115.1312 132.75246) (end 117.5262 135.14746) (width 0.25) (layer B.Cu) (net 2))
 (segment (start 115.0262 132.64746) (end 115.1312 132.75246) (width 0.25) (layer B.Cu) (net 2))
 (segment (start 179.6262 118.64746) (end 177.0462 121.22746) (width 0.25) (layer B.Cu) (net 18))
 (via (at 177.0462 132.76746) (size 0.8) (drill 0.4) (layers F.Cu B.Cu) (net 18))
 (segment (start 177.0462 124.84746) (end 177.0462 132.76746) (width 0.25) (layer B.Cu) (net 18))
 (segment (start 177.0462 121.22746) (end 177.0462 124.84746) (width 0.25) (layer B.Cu) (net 18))
 (segment (start 177.0462 132.76746) (end 169.1262 132.76746) (width 0.25) (layer F.Cu) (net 18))
 (via (at 124.2762 118.60746) (size 0.8) (drill 0.4) (layers F.Cu B.Cu) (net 1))
 (segment (start 117.5262 125.35746) (end 124.2762 118.60746) (width 0.25) (layer B.Cu) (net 1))
 (segment (start 117.5262 132.60746) (end 117.5262 125.35746) (width 0.25) (layer B.Cu) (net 1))
 (segment (start 128.1062 118.60746) (end 128.1462 118.64746) (width 0.25) (layer F.Cu) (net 1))
 (segment (start 124.2762 118.60746) (end 128.1062 118.60746) (width 0.25) (layer F.Cu) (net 1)))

